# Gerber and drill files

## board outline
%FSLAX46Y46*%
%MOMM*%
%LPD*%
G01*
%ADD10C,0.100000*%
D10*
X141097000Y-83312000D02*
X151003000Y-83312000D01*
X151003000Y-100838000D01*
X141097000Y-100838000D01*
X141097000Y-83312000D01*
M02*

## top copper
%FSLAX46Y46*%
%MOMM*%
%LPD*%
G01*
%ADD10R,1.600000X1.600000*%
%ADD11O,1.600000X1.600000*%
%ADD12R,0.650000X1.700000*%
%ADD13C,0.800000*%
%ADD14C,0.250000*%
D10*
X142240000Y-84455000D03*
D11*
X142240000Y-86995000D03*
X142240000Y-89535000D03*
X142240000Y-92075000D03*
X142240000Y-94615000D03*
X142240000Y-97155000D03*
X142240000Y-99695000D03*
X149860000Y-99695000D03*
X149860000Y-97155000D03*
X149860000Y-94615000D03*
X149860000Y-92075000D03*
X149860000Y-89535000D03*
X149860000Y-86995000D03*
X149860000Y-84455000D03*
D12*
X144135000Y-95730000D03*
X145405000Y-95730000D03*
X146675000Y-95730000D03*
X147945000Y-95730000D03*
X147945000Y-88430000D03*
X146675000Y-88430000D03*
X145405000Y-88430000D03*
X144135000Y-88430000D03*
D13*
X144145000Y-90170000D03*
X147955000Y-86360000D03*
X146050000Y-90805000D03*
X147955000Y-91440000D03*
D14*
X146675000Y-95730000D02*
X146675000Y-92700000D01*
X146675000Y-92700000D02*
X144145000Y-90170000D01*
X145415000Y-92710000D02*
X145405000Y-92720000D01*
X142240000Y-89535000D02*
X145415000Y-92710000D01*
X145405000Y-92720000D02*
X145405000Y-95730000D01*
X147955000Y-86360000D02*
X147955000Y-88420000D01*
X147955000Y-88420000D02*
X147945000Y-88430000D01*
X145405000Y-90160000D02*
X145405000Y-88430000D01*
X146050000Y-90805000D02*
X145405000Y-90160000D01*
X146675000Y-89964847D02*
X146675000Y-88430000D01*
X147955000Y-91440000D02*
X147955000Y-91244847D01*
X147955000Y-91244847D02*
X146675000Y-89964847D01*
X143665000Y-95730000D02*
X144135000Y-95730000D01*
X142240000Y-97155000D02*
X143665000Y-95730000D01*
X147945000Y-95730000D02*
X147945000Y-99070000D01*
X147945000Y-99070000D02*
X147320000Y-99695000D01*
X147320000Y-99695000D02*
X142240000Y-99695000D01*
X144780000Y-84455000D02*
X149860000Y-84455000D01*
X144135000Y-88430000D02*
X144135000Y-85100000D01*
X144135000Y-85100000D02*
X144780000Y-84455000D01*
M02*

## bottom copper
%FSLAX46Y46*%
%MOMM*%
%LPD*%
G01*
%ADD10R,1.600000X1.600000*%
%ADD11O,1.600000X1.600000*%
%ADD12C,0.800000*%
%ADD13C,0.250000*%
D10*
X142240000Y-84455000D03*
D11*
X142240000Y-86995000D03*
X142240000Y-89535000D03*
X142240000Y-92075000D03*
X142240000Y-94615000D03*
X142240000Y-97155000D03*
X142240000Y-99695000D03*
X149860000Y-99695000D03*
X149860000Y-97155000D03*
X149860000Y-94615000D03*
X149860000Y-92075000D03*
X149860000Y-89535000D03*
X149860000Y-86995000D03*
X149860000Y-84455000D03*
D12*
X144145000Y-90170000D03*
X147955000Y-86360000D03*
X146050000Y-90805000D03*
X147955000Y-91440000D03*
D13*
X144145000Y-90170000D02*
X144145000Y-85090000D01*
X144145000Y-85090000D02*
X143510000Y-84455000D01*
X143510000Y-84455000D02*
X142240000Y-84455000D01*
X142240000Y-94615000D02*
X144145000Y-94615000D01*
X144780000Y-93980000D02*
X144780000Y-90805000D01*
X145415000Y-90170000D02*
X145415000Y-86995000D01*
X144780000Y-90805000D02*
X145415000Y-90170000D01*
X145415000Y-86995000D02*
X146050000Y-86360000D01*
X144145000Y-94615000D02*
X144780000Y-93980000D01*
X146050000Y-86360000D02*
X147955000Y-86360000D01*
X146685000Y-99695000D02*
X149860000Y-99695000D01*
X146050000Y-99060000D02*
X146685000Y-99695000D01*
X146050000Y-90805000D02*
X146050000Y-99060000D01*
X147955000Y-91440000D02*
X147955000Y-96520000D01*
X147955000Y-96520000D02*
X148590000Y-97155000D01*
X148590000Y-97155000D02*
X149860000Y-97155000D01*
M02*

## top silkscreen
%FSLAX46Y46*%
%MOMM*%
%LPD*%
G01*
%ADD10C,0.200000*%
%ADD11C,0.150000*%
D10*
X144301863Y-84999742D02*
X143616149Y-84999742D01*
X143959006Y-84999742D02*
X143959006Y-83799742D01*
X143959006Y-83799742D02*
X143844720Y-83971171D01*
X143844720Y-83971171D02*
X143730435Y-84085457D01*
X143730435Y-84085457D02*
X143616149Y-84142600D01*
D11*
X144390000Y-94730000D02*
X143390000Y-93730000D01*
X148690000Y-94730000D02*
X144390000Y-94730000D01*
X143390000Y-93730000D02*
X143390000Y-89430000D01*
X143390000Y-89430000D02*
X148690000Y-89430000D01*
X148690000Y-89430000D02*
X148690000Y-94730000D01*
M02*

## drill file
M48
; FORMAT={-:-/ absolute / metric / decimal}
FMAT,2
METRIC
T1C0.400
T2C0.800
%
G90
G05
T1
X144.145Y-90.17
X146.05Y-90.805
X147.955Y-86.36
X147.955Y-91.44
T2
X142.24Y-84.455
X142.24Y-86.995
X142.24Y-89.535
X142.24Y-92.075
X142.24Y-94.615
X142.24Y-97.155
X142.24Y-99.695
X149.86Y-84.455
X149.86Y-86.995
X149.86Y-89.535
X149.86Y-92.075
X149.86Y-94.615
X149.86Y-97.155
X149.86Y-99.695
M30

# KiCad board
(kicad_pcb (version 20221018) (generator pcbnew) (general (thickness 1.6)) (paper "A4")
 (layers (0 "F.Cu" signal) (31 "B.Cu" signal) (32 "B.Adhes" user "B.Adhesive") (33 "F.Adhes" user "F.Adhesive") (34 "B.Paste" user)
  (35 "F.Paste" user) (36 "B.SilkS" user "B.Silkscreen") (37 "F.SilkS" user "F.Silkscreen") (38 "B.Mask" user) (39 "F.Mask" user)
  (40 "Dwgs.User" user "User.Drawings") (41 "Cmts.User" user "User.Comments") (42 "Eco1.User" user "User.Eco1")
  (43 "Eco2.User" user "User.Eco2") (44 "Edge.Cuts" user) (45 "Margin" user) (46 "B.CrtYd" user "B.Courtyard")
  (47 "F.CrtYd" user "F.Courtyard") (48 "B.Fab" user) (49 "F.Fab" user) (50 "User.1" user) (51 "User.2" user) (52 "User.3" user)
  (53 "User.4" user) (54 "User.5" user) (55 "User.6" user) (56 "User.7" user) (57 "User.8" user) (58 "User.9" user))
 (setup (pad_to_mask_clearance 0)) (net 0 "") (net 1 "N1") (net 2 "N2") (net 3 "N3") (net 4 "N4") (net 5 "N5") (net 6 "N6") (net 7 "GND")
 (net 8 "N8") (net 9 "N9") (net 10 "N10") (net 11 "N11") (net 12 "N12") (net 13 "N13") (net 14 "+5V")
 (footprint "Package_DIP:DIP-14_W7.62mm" (layer "F.Cu") (at 142.24 84.455)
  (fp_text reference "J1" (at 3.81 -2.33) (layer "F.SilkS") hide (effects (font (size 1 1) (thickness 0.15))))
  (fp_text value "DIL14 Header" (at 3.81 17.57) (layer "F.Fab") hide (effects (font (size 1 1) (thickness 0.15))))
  (pad "1" thru_hole rect (at 0 0) (size 1.6 1.6) (drill 0.8) (layers "*.Cu" "*.Mask") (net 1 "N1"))
  (pad "2" thru_hole oval (at 0 2.54) (size 1.6 1.6) (drill 0.8) (layers "*.Cu" "*.Mask") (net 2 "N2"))
  (pad "3" thru_hole oval (at 0 5.08) (size 1.6 1.6) (drill 0.8) (layers "*.Cu" "*.Mask") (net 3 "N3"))
  (pad "4" thru_hole oval (at 0 7.62) (size 1.6 1.6) (drill 0.8) (layers "*.Cu" "*.Mask") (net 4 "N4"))
  (pad "5" thru_hole oval (at 0 10.16) (size 1.6 1.6) (drill 0.8) (layers "*.Cu" "*.Mask") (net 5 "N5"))
  (pad "6" thru_hole oval (at 0 12.7) (size 1.6 1.6) (drill 0.8) (layers "*.Cu" "*.Mask") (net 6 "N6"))
  (pad "7" thru_hole oval (at 0 15.24) (size 1.6 1.6) (drill 0.8) (layers "*.Cu" "*.Mask") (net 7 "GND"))
  (pad "8" thru_hole oval (at 7.62 15.24) (size 1.6 1.6) (drill 0.8) (layers "*.Cu" "*.Mask") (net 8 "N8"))
  (pad "9" thru_hole oval (at 7.62 12.7) (size 1.6 1.6) (drill 0.8) (layers "*.Cu" "*.Mask") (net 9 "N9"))
  (pad "10" thru_hole oval (at 7.62 10.16) (size 1.6 1.6) (drill 0.8) (layers "*.Cu" "*.Mask") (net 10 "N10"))
  (pad "11" thru_hole oval (at 7.62 7.62) (size 1.6 1.6) (drill 0.8) (layers "*.Cu" "*.Mask") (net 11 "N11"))
  (pad "12" thru_hole oval (at 7.62 5.08) (size 1.6 1.6) (drill 0.8) (layers "*.Cu" "*.Mask") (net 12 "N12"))
  (pad "13" thru_hole oval (at 7.62 2.54) (size 1.6 1.6) (drill 0.8) (layers "*.Cu" "*.Mask") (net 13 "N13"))
  (pad "14" thru_hole oval (at 7.62 0) (size 1.6 1.6) (drill 0.8) (layers "*.Cu" "*.Mask") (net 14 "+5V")))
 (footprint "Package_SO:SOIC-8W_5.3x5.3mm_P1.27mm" (layer "F.Cu") (at 146.04 92.08 90)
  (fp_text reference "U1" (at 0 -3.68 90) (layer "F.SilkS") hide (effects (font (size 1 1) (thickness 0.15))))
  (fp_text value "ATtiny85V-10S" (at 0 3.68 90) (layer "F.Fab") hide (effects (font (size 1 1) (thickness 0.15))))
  (fp_line (start -2.65 -1.65) (end -1.65 -2.65) (stroke (width 0.15) (type solid)) (layer "F.SilkS"))
  (fp_line (start -2.65 2.65) (end -2.65 -1.65) (stroke (width 0.15) (type solid)) (layer "F.SilkS"))
  (fp_line (start -1.65 -2.65) (end 2.65 -2.65) (stroke (width 0.15) (type solid)) (layer "F.SilkS"))
  (fp_line (start 2.65 -2.65) (end 2.65 2.65) (stroke (width 0.15) (type solid)) (layer "F.SilkS"))
  (fp_line (start 2.65 2.65) (end -2.65 2.65) (stroke (width 0.15) (type solid)) (layer "F.SilkS"))
  (pad "1" smd rect (at -3.65 -1.905 90) (size 1.7 0.65) (layers "F.Cu" "F.Paste" "F.Mask") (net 6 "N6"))
  (pad "2" smd rect (at -3.65 -0.635 90) (size 1.7 0.65) (layers "F.Cu" "F.Paste" "F.Mask") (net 3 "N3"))
  (pad "3" smd rect (at -3.65 0.635 90) (size 1.7 0.65) (layers "F.Cu" "F.Paste" "F.Mask") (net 1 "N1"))
  (pad "4" smd rect (at -3.65 1.905 90) (size 1.7 0.65) (layers "F.Cu" "F.Paste" "F.Mask") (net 7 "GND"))
  (pad "5" smd rect (at 3.65 1.905 90) (size 1.7 0.65) (layers "F.Cu" "F.Paste" "F.Mask") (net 5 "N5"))
  (pad "6" smd rect (at 3.65 0.635 90) (size 1.7 0.65) (layers "F.Cu" "F.Paste" "F.Mask") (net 9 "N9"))
  (pad "7" smd rect (at 3.65 -0.635 90) (size 1.7 0.65) (layers "F.Cu" "F.Paste" "F.Mask") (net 8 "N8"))
  (pad "8" smd rect (at 3.65 -1.905 90) (size 1.7 0.65) (layers "F.Cu" "F.Paste" "F.Mask") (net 14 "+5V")))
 (gr_rect (start 141.097 83.312) (end 151.003 100.838) (stroke (width 0.1) (type default)) (fill none) (layer "Edge.Cuts"))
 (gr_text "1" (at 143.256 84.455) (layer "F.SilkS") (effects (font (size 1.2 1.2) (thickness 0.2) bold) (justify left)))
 (segment (start 146.675 95.73) (end 146.675 92.7) (width 0.25) (layer "F.Cu") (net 1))
 (segment (start 146.675 92.7) (end 144.145 90.17) (width 0.25) (layer "F.Cu") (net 1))
 (via (at 144.145 90.17) (size 0.8) (drill 0.4) (layers "F.Cu" "B.Cu") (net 1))
 (segment (start 144.145 90.17) (end 144.145 85.09) (width 0.25) (layer "B.Cu") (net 1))
 (segment (start 144.145 85.09) (end 143.51 84.455) (width 0.25) (layer "B.Cu") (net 1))
 (segment (start 143.51 84.455) (end 142.24 84.455) (width 0.25) (layer "B.Cu") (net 1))
 (segment (start 145.415 92.71) (end 145.405 92.72) (width 0.25) (layer "F.Cu") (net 3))
 (segment (start 142.24 89.535) (end 145.415 92.71) (width 0.25) (layer "F.Cu") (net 3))
 (segment (start 145.405 92.72) (end 145.405 95.73) (width 0.25) (layer "F.Cu") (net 3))
 (segment (start 147.955 86.36) (end 147.955 88.42) (width 0.25) (layer "F.Cu") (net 5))
 (segment (start 147.955 88.42) (end 147.945 88.43) (width 0.25) (layer "F.Cu") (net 5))
 (via (at 147.955 86.36) (size 0.8) (drill 0.4) (layers "F.Cu" "B.Cu") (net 5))
 (segment (start 142.24 94.615) (end 144.145 94.615) (width 0.25) (layer "B.Cu") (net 5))
 (segment (start 144.78 93.98) (end 144.78 90.805) (width 0.25) (layer "B.Cu") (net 5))
 (segment (start 145.415 90.17) (end 145.415 86.995) (width 0.25) (layer "B.Cu") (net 5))
 (segment (start 144.78 90.805) (end 145.415 90.17) (width 0.25) (layer "B.Cu") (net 5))
 (segment (start 145.415 86.995) (end 146.05 86.36) (width 0.25) (layer "B.Cu") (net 5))
 (segment (start 144.145 94.615) (end 144.78 93.98) (width 0.25) (layer "B.Cu") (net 5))
 (segment (start 146.05 86.36) (end 147.955 86.36) (width 0.25) (layer "B.Cu") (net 5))
 (segment (start 145.405 90.16) (end 145.405 88.43) (width 0.25) (layer "F.Cu") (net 8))
 (segment (start 146.05 90.805) (end 145.405 90.16) (width 0.25) (layer "F.Cu") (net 8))
 (via (at 146.05 90.805) (size 0.8) (drill 0.4) (layers "F.Cu" "B.Cu") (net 8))
 (segment (start 146.685 99.695) (end 149.86 99.695) (width 0.25) (layer "B.Cu") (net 8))
 (segment (start 146.05 99.06) (end 146.685 99.695) (width 0.25) (layer "B.Cu") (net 8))
 (segment (start 146.05 90.805) (end 146.05 99.06) (width 0.25) (layer "B.Cu") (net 8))
 (segment (start 146.675 89.964847) (end 146.675 88.43) (width 0.25) (layer "F.Cu") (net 9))
 (segment (start 147.955 91.44) (end 147.955 91.244847) (width 0.25) (layer "F.Cu") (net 9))
 (segment (start 147.955 91.244847) (end 146.675 89.964847) (width 0.25) (layer "F.Cu") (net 9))
 (via (at 147.955 91.44) (size 0.8) (drill 0.4) (layers "F.Cu" "B.Cu") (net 9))
 (segment (start 147.955 91.44) (end 147.955 96.52) (width 0.25) (layer "B.Cu") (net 9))
 (segment (start 147.955 96.52) (end 148.59 97.155) (width 0.25) (layer "B.Cu") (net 9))
 (segment (start 148.59 97.155) (end 149.86 97.155) (width 0.25) (layer "B.Cu") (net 9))
 (segment (start 143.665 95.73) (end 144.135 95.73) (width 0.25) (layer "F.Cu") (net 6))
 (segment (start 142.24 97.155) (end 143.665 95.73) (width 0.25) (layer "F.Cu") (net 6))
 (segment (start 147.945 95.73) (end 147.945 99.07) (width 0.25) (layer "F.Cu") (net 7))
 (segment (start 147.945 99.07) (end 147.32 99.695) (width 0.25) (layer "F.Cu") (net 7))
 (segment (start 147.32 99.695) (end 142.24 99.695) (width 0.25) (layer "F.Cu") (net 7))
 (segment (start 144.78 84.455) (end 149.86 84.455) (width 0.25) (layer "F.Cu") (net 14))
 (segment (start 144.135 88.43) (end 144.135 85.1) (width 0.25) (layer "F.Cu") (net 14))
 (segment (start 144.135 85.1) (end 144.78 84.455) (width 0.25) (layer "F.Cu") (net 14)))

